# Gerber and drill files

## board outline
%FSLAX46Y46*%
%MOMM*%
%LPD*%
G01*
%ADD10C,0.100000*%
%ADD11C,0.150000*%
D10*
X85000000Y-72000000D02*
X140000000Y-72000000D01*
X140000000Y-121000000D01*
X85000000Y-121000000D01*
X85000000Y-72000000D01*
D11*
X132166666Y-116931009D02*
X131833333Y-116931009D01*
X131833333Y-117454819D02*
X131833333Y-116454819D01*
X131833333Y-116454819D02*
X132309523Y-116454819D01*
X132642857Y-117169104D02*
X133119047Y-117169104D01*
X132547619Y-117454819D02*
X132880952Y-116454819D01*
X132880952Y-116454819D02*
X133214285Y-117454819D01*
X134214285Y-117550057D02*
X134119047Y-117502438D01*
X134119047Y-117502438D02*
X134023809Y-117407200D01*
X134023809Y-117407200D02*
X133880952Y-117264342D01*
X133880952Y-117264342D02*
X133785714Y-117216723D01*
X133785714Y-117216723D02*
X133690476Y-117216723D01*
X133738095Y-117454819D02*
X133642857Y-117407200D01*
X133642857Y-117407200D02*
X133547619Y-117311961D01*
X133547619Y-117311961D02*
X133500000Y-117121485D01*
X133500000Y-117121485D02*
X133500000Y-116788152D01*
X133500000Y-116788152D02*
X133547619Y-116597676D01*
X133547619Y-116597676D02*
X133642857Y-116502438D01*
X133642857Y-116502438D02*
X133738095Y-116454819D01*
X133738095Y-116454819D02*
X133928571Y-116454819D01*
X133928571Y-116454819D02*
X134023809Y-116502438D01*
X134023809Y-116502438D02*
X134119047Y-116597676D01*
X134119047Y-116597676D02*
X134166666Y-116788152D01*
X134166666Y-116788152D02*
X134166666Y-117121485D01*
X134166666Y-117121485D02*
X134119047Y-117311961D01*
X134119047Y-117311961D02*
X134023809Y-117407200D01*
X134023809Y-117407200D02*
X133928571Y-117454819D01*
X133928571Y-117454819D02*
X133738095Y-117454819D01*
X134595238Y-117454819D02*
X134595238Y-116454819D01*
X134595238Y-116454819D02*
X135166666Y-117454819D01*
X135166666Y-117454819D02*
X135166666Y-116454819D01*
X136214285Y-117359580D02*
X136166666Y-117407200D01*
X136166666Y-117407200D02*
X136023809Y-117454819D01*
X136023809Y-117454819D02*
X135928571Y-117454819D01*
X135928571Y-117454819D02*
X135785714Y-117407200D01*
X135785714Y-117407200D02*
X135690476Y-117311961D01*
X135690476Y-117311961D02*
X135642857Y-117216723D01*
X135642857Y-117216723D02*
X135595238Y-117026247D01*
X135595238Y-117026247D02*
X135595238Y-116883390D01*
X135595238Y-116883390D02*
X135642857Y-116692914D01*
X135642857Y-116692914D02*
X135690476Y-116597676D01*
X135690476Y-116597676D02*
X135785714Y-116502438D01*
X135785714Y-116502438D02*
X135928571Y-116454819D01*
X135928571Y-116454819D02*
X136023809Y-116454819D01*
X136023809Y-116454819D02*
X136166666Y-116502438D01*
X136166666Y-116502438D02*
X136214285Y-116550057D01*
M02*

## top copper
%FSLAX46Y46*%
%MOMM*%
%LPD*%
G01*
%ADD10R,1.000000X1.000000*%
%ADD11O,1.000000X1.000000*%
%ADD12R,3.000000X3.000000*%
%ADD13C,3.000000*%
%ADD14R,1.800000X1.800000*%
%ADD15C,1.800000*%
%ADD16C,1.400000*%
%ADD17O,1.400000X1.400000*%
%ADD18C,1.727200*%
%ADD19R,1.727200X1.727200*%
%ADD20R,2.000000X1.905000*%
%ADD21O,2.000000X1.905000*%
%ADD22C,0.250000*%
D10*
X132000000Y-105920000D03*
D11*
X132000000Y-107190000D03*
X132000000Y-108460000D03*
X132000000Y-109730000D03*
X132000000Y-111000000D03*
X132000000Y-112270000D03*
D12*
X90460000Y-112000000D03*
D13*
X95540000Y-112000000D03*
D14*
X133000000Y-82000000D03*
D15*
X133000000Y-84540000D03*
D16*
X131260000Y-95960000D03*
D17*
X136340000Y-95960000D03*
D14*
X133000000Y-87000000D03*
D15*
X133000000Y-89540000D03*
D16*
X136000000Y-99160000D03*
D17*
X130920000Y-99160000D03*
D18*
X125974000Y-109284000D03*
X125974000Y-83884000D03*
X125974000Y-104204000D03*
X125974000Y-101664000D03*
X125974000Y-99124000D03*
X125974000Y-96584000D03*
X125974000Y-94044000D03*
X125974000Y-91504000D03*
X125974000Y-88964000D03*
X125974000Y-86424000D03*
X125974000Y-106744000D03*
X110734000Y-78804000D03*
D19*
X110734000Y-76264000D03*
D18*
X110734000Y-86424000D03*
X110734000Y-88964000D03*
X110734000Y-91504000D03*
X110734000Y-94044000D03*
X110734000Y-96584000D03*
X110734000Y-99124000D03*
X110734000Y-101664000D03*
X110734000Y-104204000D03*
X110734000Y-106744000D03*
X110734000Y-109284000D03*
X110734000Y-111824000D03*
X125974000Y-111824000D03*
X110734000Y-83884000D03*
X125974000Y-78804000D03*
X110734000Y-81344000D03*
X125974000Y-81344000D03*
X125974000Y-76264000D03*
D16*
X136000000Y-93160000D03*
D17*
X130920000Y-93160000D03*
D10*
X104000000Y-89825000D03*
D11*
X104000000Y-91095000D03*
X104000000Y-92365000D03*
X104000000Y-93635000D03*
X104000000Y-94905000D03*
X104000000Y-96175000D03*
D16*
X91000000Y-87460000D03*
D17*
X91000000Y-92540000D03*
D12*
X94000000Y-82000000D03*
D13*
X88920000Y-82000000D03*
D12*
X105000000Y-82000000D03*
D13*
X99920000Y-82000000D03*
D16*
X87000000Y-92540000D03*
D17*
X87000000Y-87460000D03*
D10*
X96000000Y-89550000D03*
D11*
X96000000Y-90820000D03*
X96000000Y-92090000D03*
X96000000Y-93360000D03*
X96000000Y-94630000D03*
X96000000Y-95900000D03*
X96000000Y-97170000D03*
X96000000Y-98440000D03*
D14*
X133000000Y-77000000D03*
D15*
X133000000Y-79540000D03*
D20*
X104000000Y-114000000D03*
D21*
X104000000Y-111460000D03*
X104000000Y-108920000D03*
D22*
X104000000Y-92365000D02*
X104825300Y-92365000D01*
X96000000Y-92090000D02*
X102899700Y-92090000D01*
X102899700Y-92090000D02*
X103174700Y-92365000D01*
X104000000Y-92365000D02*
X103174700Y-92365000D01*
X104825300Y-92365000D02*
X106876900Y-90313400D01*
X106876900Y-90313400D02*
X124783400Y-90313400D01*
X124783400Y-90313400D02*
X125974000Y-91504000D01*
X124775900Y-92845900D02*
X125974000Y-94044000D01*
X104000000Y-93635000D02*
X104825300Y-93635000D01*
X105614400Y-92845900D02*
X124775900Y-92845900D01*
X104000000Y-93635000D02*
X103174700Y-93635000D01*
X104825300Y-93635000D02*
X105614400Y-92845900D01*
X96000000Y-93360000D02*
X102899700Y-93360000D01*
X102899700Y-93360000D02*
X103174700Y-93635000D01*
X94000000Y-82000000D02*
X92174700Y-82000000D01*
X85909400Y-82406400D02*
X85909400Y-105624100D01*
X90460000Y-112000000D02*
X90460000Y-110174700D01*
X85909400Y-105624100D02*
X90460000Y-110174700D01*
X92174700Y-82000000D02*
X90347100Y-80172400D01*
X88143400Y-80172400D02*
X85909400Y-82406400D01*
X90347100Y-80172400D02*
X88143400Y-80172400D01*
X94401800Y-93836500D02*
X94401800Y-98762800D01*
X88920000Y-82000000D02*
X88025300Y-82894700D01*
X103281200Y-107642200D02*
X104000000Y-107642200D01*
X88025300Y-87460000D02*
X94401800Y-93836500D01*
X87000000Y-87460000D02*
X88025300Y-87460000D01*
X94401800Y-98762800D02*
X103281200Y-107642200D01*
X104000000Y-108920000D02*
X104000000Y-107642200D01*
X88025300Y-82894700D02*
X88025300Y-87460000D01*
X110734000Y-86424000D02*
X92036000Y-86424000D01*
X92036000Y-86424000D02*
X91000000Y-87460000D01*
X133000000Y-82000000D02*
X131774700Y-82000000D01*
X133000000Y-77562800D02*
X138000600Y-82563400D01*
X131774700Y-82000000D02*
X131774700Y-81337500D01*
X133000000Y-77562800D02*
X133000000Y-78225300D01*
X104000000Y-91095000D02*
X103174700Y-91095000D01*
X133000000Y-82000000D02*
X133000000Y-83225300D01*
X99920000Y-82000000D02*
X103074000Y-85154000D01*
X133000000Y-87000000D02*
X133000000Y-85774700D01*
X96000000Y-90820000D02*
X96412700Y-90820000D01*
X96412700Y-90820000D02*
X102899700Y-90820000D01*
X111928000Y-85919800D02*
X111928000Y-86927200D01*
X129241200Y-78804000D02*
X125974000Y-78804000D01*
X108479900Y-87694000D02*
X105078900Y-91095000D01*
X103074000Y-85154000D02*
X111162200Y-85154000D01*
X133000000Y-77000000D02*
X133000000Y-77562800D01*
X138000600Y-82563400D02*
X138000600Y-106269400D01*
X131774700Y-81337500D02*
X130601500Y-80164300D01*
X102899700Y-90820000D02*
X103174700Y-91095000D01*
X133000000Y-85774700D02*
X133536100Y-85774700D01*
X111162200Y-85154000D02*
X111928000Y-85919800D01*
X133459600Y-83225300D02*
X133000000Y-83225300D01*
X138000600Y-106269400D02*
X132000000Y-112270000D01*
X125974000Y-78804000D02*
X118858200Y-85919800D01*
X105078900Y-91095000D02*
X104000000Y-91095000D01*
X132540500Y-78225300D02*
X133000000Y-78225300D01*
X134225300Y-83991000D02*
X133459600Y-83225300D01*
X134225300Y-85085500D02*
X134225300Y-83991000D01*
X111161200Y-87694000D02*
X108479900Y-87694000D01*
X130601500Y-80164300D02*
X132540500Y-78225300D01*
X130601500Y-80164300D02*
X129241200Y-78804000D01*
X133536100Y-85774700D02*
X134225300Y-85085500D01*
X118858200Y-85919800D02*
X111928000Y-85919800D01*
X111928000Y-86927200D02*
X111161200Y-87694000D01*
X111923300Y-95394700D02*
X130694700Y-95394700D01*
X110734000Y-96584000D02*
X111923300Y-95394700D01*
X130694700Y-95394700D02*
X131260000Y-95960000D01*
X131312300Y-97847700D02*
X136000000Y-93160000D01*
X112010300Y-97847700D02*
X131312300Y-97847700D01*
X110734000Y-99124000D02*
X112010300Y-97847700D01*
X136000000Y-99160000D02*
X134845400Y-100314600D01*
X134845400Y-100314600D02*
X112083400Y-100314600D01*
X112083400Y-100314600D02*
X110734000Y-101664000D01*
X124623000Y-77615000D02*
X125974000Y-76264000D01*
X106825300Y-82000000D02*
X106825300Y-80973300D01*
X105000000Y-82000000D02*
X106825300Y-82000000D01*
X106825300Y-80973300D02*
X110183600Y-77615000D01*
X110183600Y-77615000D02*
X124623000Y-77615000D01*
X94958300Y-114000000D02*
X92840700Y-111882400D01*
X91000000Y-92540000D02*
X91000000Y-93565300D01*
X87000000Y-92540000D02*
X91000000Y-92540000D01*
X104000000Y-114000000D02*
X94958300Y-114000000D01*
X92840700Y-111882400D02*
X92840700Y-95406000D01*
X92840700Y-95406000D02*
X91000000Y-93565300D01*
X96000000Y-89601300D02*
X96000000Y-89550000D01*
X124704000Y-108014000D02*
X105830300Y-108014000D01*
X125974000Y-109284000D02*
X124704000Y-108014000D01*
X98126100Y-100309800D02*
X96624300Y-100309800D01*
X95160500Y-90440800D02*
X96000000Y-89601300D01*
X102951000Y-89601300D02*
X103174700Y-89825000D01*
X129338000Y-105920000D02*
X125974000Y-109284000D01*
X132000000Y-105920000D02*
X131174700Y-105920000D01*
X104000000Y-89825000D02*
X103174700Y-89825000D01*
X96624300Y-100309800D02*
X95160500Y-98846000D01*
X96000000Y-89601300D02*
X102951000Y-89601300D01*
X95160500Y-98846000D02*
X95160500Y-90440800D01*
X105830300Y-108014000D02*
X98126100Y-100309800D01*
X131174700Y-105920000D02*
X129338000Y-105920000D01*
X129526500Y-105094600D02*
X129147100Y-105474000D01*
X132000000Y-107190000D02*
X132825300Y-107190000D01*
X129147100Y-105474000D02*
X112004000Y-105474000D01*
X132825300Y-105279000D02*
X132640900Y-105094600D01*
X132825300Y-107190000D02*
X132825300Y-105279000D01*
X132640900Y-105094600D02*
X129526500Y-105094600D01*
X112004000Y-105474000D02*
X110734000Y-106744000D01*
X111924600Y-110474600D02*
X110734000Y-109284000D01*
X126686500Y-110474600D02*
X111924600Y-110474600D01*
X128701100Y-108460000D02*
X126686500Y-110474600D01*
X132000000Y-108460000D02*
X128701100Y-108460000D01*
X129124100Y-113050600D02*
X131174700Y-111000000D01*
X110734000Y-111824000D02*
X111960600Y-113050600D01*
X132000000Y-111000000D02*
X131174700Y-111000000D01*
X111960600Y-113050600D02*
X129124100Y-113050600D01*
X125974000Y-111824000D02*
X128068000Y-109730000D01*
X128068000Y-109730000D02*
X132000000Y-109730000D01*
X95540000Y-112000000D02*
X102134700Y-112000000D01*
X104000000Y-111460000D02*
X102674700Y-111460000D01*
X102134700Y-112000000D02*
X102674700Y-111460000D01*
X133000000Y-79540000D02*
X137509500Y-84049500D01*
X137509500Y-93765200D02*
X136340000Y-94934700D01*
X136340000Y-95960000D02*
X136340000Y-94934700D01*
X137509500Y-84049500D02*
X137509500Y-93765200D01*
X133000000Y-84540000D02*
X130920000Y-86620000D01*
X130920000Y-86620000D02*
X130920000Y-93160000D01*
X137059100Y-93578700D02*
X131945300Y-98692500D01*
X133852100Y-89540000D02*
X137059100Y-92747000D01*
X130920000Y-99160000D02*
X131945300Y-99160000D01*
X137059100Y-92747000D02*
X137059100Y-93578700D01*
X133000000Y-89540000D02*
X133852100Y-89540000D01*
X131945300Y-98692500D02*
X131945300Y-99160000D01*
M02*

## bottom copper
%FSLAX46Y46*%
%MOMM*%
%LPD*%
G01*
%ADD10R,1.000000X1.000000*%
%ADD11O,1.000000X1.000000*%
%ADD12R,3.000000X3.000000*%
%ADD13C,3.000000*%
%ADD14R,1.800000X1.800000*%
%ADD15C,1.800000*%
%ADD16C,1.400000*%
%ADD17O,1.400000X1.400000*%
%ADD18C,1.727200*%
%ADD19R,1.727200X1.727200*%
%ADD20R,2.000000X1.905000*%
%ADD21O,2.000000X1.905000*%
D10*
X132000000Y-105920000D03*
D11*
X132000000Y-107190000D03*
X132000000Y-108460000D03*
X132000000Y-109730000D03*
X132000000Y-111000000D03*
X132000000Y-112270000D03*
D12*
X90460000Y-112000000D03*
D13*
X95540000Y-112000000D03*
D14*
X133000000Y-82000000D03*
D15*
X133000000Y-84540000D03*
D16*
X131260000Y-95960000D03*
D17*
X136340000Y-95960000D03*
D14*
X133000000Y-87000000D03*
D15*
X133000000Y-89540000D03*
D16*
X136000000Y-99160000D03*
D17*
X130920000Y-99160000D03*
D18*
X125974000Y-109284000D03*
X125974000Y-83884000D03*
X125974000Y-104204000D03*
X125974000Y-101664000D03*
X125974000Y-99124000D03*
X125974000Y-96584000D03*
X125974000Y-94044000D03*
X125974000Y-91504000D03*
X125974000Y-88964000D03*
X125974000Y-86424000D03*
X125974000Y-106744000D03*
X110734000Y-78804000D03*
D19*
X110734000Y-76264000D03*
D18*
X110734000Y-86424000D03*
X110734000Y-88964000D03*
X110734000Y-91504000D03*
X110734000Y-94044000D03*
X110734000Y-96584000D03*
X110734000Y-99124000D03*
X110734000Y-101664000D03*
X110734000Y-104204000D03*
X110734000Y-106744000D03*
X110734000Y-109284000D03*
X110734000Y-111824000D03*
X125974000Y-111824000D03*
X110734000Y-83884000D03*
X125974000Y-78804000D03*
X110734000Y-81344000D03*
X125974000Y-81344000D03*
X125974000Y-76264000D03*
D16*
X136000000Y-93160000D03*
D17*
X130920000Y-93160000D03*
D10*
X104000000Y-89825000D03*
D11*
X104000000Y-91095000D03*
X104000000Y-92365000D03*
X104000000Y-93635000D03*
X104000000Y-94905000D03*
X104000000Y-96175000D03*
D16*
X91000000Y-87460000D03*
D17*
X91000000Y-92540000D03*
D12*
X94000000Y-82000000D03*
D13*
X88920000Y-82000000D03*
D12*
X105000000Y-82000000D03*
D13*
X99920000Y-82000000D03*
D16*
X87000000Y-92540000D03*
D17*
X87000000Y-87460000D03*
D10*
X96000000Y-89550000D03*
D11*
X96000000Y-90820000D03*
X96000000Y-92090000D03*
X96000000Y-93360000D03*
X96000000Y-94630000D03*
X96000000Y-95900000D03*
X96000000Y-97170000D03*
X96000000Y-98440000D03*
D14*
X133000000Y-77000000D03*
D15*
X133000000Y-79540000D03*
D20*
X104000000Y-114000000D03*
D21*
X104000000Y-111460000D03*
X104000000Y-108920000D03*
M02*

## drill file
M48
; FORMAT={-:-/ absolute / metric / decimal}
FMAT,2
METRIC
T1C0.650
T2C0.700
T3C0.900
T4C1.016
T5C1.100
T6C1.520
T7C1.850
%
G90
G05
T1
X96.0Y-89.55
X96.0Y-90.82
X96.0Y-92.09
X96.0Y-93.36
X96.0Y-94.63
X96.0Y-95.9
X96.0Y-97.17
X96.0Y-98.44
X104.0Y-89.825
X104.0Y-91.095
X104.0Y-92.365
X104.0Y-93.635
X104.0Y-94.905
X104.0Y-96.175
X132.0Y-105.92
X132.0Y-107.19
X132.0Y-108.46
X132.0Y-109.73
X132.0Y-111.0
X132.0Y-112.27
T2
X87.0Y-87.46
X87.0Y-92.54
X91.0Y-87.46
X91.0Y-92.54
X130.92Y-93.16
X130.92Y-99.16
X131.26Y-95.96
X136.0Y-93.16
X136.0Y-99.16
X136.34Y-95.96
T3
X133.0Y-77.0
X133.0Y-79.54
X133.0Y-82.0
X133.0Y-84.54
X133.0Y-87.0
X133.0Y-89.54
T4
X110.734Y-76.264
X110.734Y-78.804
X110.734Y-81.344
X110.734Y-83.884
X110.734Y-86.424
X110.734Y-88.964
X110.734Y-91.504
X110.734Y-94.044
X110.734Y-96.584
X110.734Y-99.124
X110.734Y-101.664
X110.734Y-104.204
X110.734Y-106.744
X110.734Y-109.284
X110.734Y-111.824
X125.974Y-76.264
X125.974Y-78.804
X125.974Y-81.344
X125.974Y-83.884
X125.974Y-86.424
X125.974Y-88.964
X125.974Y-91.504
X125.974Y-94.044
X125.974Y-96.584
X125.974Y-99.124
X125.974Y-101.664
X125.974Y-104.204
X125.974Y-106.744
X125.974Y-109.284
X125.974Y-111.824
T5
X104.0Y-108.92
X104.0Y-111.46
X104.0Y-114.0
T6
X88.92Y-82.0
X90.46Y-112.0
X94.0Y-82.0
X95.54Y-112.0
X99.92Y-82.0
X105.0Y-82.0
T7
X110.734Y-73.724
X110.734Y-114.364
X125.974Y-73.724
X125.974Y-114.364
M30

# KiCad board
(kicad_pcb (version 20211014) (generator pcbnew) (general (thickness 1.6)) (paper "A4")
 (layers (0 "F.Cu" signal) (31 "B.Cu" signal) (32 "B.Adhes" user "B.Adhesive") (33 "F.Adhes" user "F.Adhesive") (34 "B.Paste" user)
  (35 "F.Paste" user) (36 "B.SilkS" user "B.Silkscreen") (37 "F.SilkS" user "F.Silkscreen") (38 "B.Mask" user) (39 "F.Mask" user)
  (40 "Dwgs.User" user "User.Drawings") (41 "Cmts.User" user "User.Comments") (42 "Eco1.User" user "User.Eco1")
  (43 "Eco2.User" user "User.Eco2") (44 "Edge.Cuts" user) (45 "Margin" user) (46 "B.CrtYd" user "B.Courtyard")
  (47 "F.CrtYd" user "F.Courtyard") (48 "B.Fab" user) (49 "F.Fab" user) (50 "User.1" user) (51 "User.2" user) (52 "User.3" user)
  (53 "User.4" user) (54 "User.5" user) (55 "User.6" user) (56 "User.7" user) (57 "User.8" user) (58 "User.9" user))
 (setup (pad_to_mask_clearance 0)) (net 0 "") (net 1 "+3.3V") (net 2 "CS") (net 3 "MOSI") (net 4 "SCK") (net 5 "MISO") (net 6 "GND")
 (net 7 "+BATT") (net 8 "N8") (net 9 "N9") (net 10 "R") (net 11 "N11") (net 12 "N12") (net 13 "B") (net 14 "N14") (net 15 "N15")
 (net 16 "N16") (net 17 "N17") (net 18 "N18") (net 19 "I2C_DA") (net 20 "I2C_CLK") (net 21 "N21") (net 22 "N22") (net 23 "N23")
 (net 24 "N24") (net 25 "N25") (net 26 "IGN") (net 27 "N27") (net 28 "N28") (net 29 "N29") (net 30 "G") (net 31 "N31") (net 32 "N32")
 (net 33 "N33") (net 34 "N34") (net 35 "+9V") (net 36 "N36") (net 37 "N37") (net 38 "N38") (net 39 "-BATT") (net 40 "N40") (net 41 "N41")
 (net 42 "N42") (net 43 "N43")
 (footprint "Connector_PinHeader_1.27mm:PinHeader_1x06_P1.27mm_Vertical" (layer "F.Cu") (at 132 105.92)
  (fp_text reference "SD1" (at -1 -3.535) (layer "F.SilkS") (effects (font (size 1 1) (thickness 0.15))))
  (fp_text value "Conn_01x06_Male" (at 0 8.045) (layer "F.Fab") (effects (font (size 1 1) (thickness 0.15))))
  (pad "1" thru_hole rect (at 0 0) (size 1 1) (drill 0.65) (layers *.Cu *.Mask) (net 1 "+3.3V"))
  (pad "2" thru_hole oval (at 0 1.27) (size 1 1) (drill 0.65) (layers *.Cu *.Mask) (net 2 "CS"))
  (pad "3" thru_hole oval (at 0 2.54) (size 1 1) (drill 0.65) (layers *.Cu *.Mask) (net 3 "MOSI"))
  (pad "4" thru_hole oval (at 0 3.81) (size 1 1) (drill 0.65) (layers *.Cu *.Mask) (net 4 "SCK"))
  (pad "5" thru_hole oval (at 0 5.08) (size 1 1) (drill 0.65) (layers *.Cu *.Mask) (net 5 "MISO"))
  (pad "6" thru_hole oval (at 0 6.35) (size 1 1) (drill 0.65) (layers *.Cu *.Mask) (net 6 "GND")))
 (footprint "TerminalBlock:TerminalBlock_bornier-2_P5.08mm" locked (layer "F.Cu") (at 90.46 112)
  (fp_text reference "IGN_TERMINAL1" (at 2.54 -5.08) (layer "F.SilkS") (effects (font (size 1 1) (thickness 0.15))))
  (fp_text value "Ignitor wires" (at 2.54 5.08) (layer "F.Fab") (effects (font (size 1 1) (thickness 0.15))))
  (pad "1" thru_hole rect locked (at 0 0) (size 3 3) (drill 1.52) (layers *.Cu *.Mask) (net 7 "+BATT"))
  (pad "2" thru_hole circle locked (at 5.08 0) (size 3 3) (drill 1.52) (layers *.Cu *.Mask) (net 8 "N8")))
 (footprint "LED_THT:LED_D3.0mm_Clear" (layer "F.Cu") (at 133 82 -90)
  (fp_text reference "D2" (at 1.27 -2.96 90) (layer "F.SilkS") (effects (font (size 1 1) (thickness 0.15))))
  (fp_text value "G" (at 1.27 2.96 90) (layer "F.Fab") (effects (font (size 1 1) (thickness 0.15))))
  (pad "1" thru_hole rect (at 0 0 270) (size 1.8 1.8) (drill 0.9) (layers *.Cu *.Mask) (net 6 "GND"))
  (pad "2" thru_hole circle (at 2.54 0 270) (size 1.8 1.8) (drill 0.9) (layers *.Cu *.Mask) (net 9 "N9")))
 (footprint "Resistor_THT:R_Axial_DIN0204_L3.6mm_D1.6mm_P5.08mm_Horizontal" (layer "F.Cu") (at 131.26 95.96)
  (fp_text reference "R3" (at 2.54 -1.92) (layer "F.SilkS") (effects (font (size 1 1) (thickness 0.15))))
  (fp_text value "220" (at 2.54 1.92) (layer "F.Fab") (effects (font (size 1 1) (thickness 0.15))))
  (pad "1" thru_hole circle (at 0 0) (size 1.4 1.4) (drill 0.7) (layers *.Cu *.Mask) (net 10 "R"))
  (pad "2" thru_hole oval (at 5.08 0) (size 1.4 1.4) (drill 0.7) (layers *.Cu *.Mask) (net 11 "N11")))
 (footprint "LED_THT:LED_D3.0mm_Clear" (layer "F.Cu") (at 133 87 -90)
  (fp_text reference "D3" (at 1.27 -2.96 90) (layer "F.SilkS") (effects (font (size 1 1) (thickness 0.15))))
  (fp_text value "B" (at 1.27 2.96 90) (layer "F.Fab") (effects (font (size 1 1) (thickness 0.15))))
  (pad "1" thru_hole rect (at 0 0 270) (size 1.8 1.8) (drill 0.9) (layers *.Cu *.Mask) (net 6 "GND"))
  (pad "2" thru_hole circle (at 2.54 0 270) (size 1.8 1.8) (drill 0.9) (layers *.Cu *.Mask) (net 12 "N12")))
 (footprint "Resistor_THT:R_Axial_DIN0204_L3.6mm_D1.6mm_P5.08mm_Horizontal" (layer "F.Cu") (at 136 99.16 180)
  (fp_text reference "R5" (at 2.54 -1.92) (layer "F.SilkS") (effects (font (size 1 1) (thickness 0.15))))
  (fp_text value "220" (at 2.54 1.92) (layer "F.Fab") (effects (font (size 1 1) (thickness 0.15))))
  (pad "1" thru_hole circle (at 0 0 180) (size 1.4 1.4) (drill 0.7) (layers *.Cu *.Mask) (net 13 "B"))
  (pad "2" thru_hole oval (at 5.08 0 180) (size 1.4 1.4) (drill 0.7) (layers *.Cu *.Mask) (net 12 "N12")))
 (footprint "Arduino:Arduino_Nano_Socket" (layer "F.Cu") (at 118.354 115.634)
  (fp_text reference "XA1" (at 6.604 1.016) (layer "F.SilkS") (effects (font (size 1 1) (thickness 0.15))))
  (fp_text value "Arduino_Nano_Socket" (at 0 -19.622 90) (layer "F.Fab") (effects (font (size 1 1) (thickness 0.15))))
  (pad "" np_thru_hole circle locked (at 7.62 -41.91) (size 1.85 1.85) (drill 1.85) (layers *.Cu *.Mask))
  (pad "" np_thru_hole circle locked (at 7.62 -1.27) (size 1.85 1.85) (drill 1.85) (layers *.Cu *.Mask))
  (pad "" np_thru_hole circle locked (at -7.62 -41.91) (size 1.85 1.85) (drill 1.85) (layers *.Cu *.Mask))
  (pad "" np_thru_hole circle locked (at -7.62 -1.27) (size 1.85 1.85) (drill 1.85) (layers *.Cu *.Mask))
  (pad "3V3" thru_hole circle locked (at 7.62 -6.35) (size 1.7272 1.7272) (drill 1.016) (layers *.Cu *.Mask) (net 1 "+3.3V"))
  (pad "5V" thru_hole circle locked (at 7.62 -31.75) (size 1.7272 1.7272) (drill 1.016) (layers *.Cu *.Mask) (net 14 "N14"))
  (pad "A0" thru_hole circle locked (at 7.62 -11.43) (size 1.7272 1.7272) (drill 1.016) (layers *.Cu *.Mask) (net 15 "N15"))
  (pad "A1" thru_hole circle locked (at 7.62 -13.97) (size 1.7272 1.7272) (drill 1.016) (layers *.Cu *.Mask) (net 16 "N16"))
  (pad "A2" thru_hole circle locked (at 7.62 -16.51) (size 1.7272 1.7272) (drill 1.016) (layers *.Cu *.Mask) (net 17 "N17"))
  (pad "A3" thru_hole circle locked (at 7.62 -19.05) (size 1.7272 1.7272) (drill 1.016) (layers *.Cu *.Mask) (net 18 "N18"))
  (pad "A4" thru_hole circle locked (at 7.62 -21.59) (size 1.7272 1.7272) (drill 1.016) (layers *.Cu *.Mask) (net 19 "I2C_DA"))
  (pad "A5" thru_hole circle locked (at 7.62 -24.13) (size 1.7272 1.7272) (drill 1.016) (layers *.Cu *.Mask) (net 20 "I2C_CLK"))
  (pad "A6" thru_hole circle locked (at 7.62 -26.67) (size 1.7272 1.7272) (drill 1.016) (layers *.Cu *.Mask) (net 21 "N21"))
  (pad "A7" thru_hole circle locked (at 7.62 -29.21) (size 1.7272 1.7272) (drill 1.016) (layers *.Cu *.Mask) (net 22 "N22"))
  (pad "AREF" thru_hole circle locked (at 7.62 -8.89) (size 1.7272 1.7272) (drill 1.016) (layers *.Cu *.Mask) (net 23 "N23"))
  (pad "D0" thru_hole circle locked (at -7.62 -36.83) (size 1.7272 1.7272) (drill 1.016) (layers *.Cu *.Mask) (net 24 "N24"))
  (pad "D1" thru_hole rect locked (at -7.62 -39.37) (size 1.7272 1.7272) (drill 1.016) (layers *.Cu *.Mask) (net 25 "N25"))
  (pad "D2" thru_hole circle locked (at -7.62 -29.21) (size 1.7272 1.7272) (drill 1.016) (layers *.Cu *.Mask) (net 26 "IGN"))
  (pad "D3" thru_hole circle locked (at -7.62 -26.67) (size 1.7272 1.7272) (drill 1.016) (layers *.Cu *.Mask) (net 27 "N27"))
  (pad "D4" thru_hole circle locked (at -7.62 -24.13) (size 1.7272 1.7272) (drill 1.016) (layers *.Cu *.Mask) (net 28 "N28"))
  (pad "D5" thru_hole circle locked (at -7.62 -21.59) (size 1.7272 1.7272) (drill 1.016) (layers *.Cu *.Mask) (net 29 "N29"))
  (pad "D6" thru_hole circle locked (at -7.62 -19.05) (size 1.7272 1.7272) (drill 1.016) (layers *.Cu *.Mask) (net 10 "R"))
  (pad "D7" thru_hole circle locked (at -7.62 -16.51) (size 1.7272 1.7272) (drill 1.016) (layers *.Cu *.Mask) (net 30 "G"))
  (pad "D8" thru_hole circle locked (at -7.62 -13.97) (size 1.7272 1.7272) (drill 1.016) (layers *.Cu *.Mask) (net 13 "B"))
  (pad "D9" thru_hole circle locked (at -7.62 -11.43) (size 1.7272 1.7272) (drill 1.016) (layers *.Cu *.Mask) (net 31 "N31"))
  (pad "D10" thru_hole circle locked (at -7.62 -8.89) (size 1.7272 1.7272) (drill 1.016) (layers *.Cu *.Mask) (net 2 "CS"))
  (pad "D11" thru_hole circle locked (at -7.62 -6.35) (size 1.7272 1.7272) (drill 1.016) (layers *.Cu *.Mask) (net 3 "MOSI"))
  (pad "D12" thru_hole circle locked (at -7.62 -3.81) (size 1.7272 1.7272) (drill 1.016) (layers *.Cu *.Mask) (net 5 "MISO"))
  (pad "D13" thru_hole circle locked (at 7.62 -3.81) (size 1.7272 1.7272) (drill 1.016) (layers *.Cu *.Mask) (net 4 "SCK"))
  (pad "GND1" thru_hole circle locked (at -7.62 -31.75) (size 1.7272 1.7272) (drill 1.016) (layers *.Cu *.Mask) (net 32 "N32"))
  (pad "GND2" thru_hole circle locked (at 7.62 -36.83) (size 1.7272 1.7272) (drill 1.016) (layers *.Cu *.Mask) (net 6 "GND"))
  (pad "RST1" thru_hole circle locked (at -7.62 -34.29) (size 1.7272 1.7272) (drill 1.016) (layers *.Cu *.Mask) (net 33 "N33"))
  (pad "RST2" thru_hole circle locked (at 7.62 -34.29) (size 1.7272 1.7272) (drill 1.016) (layers *.Cu *.Mask) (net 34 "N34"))
  (pad "VIN" thru_hole circle locked (at 7.62 -39.37) (size 1.7272 1.7272) (drill 1.016) (layers *.Cu *.Mask) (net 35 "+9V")))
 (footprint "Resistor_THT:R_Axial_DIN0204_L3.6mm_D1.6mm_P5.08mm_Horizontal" (layer "F.Cu") (at 136 93.16 180)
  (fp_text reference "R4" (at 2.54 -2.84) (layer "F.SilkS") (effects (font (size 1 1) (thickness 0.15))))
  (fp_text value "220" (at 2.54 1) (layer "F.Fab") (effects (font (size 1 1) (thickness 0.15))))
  (pad "1" thru_hole circle (at 0 0 180) (size 1.4 1.4) (drill 0.7) (layers *.Cu *.Mask) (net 30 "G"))
  (pad "2" thru_hole oval (at 5.08 0 180) (size 1.4 1.4) (drill 0.7) (layers *.Cu *.Mask) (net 9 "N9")))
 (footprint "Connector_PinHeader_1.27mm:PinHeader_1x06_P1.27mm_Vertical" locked (layer "F.Cu") (at 104 89.825)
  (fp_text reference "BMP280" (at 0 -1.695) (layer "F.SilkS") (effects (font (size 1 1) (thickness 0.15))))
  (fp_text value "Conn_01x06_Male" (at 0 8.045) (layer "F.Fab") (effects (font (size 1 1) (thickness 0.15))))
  (pad "1" thru_hole rect locked (at 0 0) (size 1 1) (drill 0.65) (layers *.Cu *.Mask) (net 1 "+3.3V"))
  (pad "2" thru_hole oval locked (at 0 1.27) (size 1 1) (drill 0.65) (layers *.Cu *.Mask) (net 6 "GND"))
  (pad "3" thru_hole oval locked (at 0 2.54) (size 1 1) (drill 0.65) (layers *.Cu *.Mask) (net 20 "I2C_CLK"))
  (pad "4" thru_hole oval locked (at 0 3.81) (size 1 1) (drill 0.65) (layers *.Cu *.Mask) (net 19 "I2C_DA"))
  (pad "5" thru_hole oval locked (at 0 5.08) (size 1 1) (drill 0.65) (layers *.Cu *.Mask) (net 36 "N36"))
  (pad "6" thru_hole oval locked (at 0 6.35) (size 1 1) (drill 0.65) (layers *.Cu *.Mask) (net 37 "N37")))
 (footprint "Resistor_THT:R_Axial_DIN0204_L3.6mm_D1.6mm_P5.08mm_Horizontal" (layer "F.Cu") (at 91 87.46 -90)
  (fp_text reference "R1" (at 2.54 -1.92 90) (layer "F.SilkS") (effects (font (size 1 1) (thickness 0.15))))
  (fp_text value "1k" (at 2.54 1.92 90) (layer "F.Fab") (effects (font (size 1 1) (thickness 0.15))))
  (pad "1" thru_hole circle (at 0 0 270) (size 1.4 1.4) (drill 0.7) (layers *.Cu *.Mask) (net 26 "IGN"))
  (pad "2" thru_hole oval (at 5.08 0 270) (size 1.4 1.4) (drill 0.7) (layers *.Cu *.Mask) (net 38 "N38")))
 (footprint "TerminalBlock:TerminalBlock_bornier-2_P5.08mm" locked (layer "F.Cu") (at 94 82 180)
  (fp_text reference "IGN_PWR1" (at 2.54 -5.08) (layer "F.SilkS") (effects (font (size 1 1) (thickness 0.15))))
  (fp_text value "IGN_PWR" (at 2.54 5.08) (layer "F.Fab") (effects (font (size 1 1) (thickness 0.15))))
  (pad "1" thru_hole rect locked (at 0 0 180) (size 3 3) (drill 1.52) (layers *.Cu *.Mask) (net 7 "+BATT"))
  (pad "2" thru_hole circle locked (at 5.08 0 180) (size 3 3) (drill 1.52) (layers *.Cu *.Mask) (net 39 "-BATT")))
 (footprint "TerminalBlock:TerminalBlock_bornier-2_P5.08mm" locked (layer "F.Cu") (at 105 82 180)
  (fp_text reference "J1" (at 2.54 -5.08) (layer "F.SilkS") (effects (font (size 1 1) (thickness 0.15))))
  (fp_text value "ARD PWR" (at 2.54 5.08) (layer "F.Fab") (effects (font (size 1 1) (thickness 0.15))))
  (pad "1" thru_hole rect locked (at 0 0 180) (size 3 3) (drill 1.52) (layers *.Cu *.Mask) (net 35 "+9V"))
  (pad "2" thru_hole circle locked (at 5.08 0 180) (size 3 3) (drill 1.52) (layers *.Cu *.Mask) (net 6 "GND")))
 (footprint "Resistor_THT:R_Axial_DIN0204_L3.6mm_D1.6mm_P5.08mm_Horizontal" (layer "F.Cu") (at 87 92.54 90)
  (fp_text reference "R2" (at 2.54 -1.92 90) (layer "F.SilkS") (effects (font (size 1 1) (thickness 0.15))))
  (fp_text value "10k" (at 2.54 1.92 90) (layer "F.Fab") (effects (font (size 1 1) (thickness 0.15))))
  (pad "1" thru_hole circle (at 0 0 90) (size 1.4 1.4) (drill 0.7) (layers *.Cu *.Mask) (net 38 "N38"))
  (pad "2" thru_hole oval (at 5.08 0 90) (size 1.4 1.4) (drill 0.7) (layers *.Cu *.Mask) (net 39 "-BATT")))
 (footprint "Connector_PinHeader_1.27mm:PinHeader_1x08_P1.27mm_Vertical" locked (layer "F.Cu") (at 96 89.55)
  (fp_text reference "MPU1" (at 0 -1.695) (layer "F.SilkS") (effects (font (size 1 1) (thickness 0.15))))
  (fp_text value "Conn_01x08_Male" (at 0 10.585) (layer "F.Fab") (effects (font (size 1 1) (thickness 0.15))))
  (pad "1" thru_hole rect locked (at 0 0) (size 1 1) (drill 0.65) (layers *.Cu *.Mask) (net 1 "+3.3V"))
  (pad "2" thru_hole oval locked (at 0 1.27) (size 1 1) (drill 0.65) (layers *.Cu *.Mask) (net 6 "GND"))
  (pad "3" thru_hole oval locked (at 0 2.54) (size 1 1) (drill 0.65) (layers *.Cu *.Mask) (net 20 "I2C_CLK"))
  (pad "4" thru_hole oval locked (at 0 3.81) (size 1 1) (drill 0.65) (layers *.Cu *.Mask) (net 19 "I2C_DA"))
  (pad "5" thru_hole oval locked (at 0 5.08) (size 1 1) (drill 0.65) (layers *.Cu *.Mask) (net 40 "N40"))
  (pad "6" thru_hole oval locked (at 0 6.35) (size 1 1) (drill 0.65) (layers *.Cu *.Mask) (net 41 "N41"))
  (pad "7" thru_hole oval locked (at 0 7.62) (size 1 1) (drill 0.65) (layers *.Cu *.Mask) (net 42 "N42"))
  (pad "8" thru_hole oval locked (at 0 8.89) (size 1 1) (drill 0.65) (layers *.Cu *.Mask) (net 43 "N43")))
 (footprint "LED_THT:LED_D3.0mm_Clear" (layer "F.Cu") (at 133 77 -90)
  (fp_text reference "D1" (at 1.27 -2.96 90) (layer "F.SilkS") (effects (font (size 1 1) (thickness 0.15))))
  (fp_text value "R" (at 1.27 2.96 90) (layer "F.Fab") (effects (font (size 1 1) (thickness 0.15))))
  (pad "1" thru_hole rect (at 0 0 270) (size 1.8 1.8) (drill 0.9) (layers *.Cu *.Mask) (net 6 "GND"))
  (pad "2" thru_hole circle (at 2.54 0 270) (size 1.8 1.8) (drill 0.9) (layers *.Cu *.Mask) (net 11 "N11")))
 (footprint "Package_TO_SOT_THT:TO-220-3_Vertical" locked (layer "F.Cu") (at 104 114 90)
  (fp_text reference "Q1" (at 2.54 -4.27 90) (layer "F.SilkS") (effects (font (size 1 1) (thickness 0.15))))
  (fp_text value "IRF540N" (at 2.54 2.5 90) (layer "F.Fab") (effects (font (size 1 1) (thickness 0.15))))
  (pad "1" thru_hole rect locked (at 0 0 90) (size 1.905 2) (drill 1.1) (layers *.Cu *.Mask) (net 38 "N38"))
  (pad "2" thru_hole oval locked (at 2.54 0 90) (size 1.905 2) (drill 1.1) (layers *.Cu *.Mask) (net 8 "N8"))
  (pad "3" thru_hole oval locked (at 5.08 0 90) (size 1.905 2) (drill 1.1) (layers *.Cu *.Mask) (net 39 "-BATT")))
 (gr_rect (start 85 72) (end 140 121) (layer "Edge.Cuts") (width 0.1) (fill none))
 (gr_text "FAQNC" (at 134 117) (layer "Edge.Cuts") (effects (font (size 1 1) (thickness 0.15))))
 (segment (start 104 92.365) (end 104.8253 92.365) (width 0.25) (layer "F.Cu") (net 20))
 (segment (start 96 92.09) (end 102.8997 92.09) (width 0.25) (layer "F.Cu") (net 20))
 (segment (start 102.8997 92.09) (end 103.1747 92.365) (width 0.25) (layer "F.Cu") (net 20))
 (segment (start 104 92.365) (end 103.1747 92.365) (width 0.25) (layer "F.Cu") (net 20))
 (segment (start 104.8253 92.365) (end 106.8769 90.3134) (width 0.25) (layer "F.Cu") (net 20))
 (segment (start 106.8769 90.3134) (end 124.7834 90.3134) (width 0.25) (layer "F.Cu") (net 20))
 (segment (start 124.7834 90.3134) (end 125.974 91.504) (width 0.25) (layer "F.Cu") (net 20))
 (segment (start 124.7759 92.8459) (end 125.974 94.044) (width 0.25) (layer "F.Cu") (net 19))
 (segment (start 104 93.635) (end 104.8253 93.635) (width 0.25) (layer "F.Cu") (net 19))
 (segment (start 105.6144 92.8459) (end 124.7759 92.8459) (width 0.25) (layer "F.Cu") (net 19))
 (segment (start 104 93.635) (end 103.1747 93.635) (width 0.25) (layer "F.Cu") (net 19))
 (segment (start 104.8253 93.635) (end 105.6144 92.8459) (width 0.25) (layer "F.Cu") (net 19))
 (segment (start 96 93.36) (end 102.8997 93.36) (width 0.25) (layer "F.Cu") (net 19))
 (segment (start 102.8997 93.36) (end 103.1747 93.635) (width 0.25) (layer "F.Cu") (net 19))
 (segment (start 94 82) (end 92.1747 82) (width 0.25) (layer "F.Cu") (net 7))
 (segment (start 85.9094 82.4064) (end 85.9094 105.6241) (width 0.25) (layer "F.Cu") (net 7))
 (segment (start 90.46 112) (end 90.46 110.1747) (width 0.25) (layer "F.Cu") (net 7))
 (segment (start 85.9094 105.6241) (end 90.46 110.1747) (width 0.25) (layer "F.Cu") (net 7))
 (segment (start 92.1747 82) (end 90.3471 80.1724) (width 0.25) (layer "F.Cu") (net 7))
 (segment (start 88.1434 80.1724) (end 85.9094 82.4064) (width 0.25) (layer "F.Cu") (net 7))
 (segment (start 90.3471 80.1724) (end 88.1434 80.1724) (width 0.25) (layer "F.Cu") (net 7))
 (segment (start 94.4018 93.8365) (end 94.4018 98.7628) (width 0.25) (layer "F.Cu") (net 39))
 (segment (start 88.92 82) (end 88.0253 82.8947) (width 0.25) (layer "F.Cu") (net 39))
 (segment (start 103.2812 107.6422) (end 104 107.6422) (width 0.25) (layer "F.Cu") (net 39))
 (segment (start 88.0253 87.46) (end 94.4018 93.8365) (width 0.25) (layer "F.Cu") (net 39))
 (segment (start 87 87.46) (end 88.0253 87.46) (width 0.25) (layer "F.Cu") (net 39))
 (segment (start 94.4018 98.7628) (end 103.2812 107.6422) (width 0.25) (layer "F.Cu") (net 39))
 (segment (start 104 108.92) (end 104 107.6422) (width 0.25) (layer "F.Cu") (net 39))
 (segment (start 88.0253 82.8947) (end 88.0253 87.46) (width 0.25) (layer "F.Cu") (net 39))
 (segment (start 110.734 86.424) (end 92.036 86.424) (width 0.25) (layer "F.Cu") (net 26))
 (segment (start 92.036 86.424) (end 91 87.46) (width 0.25) (layer "F.Cu") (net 26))
 (segment (start 133 82) (end 131.7747 82) (width 0.25) (layer "F.Cu") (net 6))
 (segment (start 133 77.5628) (end 138.0006 82.5634) (width 0.25) (layer "F.Cu") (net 6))
 (segment (start 131.7747 82) (end 131.7747 81.3375) (width 0.25) (layer "F.Cu") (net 6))
 (segment (start 133 77.5628) (end 133 78.2253) (width 0.25) (layer "F.Cu") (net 6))
 (segment (start 104 91.095) (end 103.1747 91.095) (width 0.25) (layer "F.Cu") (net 6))
 (segment (start 133 82) (end 133 83.2253) (width 0.25) (layer "F.Cu") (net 6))
 (segment (start 99.92 82) (end 103.074 85.154) (width 0.25) (layer "F.Cu") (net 6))
 (segment (start 133 87) (end 133 85.7747) (width 0.25) (layer "F.Cu") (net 6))
 (segment (start 96 90.82) (end 96.4127 90.82) (width 0.25) (layer "F.Cu") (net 6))
 (segment (start 96.4127 90.82) (end 102.8997 90.82) (width 0.25) (layer "F.Cu") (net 6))
 (segment (start 111.928 85.9198) (end 111.928 86.9272) (width 0.25) (layer "F.Cu") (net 6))
 (segment (start 129.2412 78.804) (end 125.974 78.804) (width 0.25) (layer "F.Cu") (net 6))
 (segment (start 108.4799 87.694) (end 105.0789 91.095) (width 0.25) (layer "F.Cu") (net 6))
 (segment (start 103.074 85.154) (end 111.1622 85.154) (width 0.25) (layer "F.Cu") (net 6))
 (segment (start 133 77) (end 133 77.5628) (width 0.25) (layer "F.Cu") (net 6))
 (segment (start 138.0006 82.5634) (end 138.0006 106.2694) (width 0.25) (layer "F.Cu") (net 6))
 (segment (start 131.7747 81.3375) (end 130.6015 80.1643) (width 0.25) (layer "F.Cu") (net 6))
 (segment (start 102.8997 90.82) (end 103.1747 91.095) (width 0.25) (layer "F.Cu") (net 6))
 (segment (start 133 85.7747) (end 133.5361 85.7747) (width 0.25) (layer "F.Cu") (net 6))
 (segment (start 111.1622 85.154) (end 111.928 85.9198) (width 0.25) (layer "F.Cu") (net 6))
 (segment (start 133.4596 83.2253) (end 133 83.2253) (width 0.25) (layer "F.Cu") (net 6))
 (segment (start 138.0006 106.2694) (end 132 112.27) (width 0.25) (layer "F.Cu") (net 6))
 (segment (start 125.974 78.804) (end 118.8582 85.9198) (width 0.25) (layer "F.Cu") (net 6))
 (segment (start 105.0789 91.095) (end 104 91.095) (width 0.25) (layer "F.Cu") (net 6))
 (segment (start 132.5405 78.2253) (end 133 78.2253) (width 0.25) (layer "F.Cu") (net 6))
 (segment (start 134.2253 83.991) (end 133.4596 83.2253) (width 0.25) (layer "F.Cu") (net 6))
 (segment (start 134.2253 85.0855) (end 134.2253 83.991) (width 0.25) (layer "F.Cu") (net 6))
 (segment (start 111.1612 87.694) (end 108.4799 87.694) (width 0.25) (layer "F.Cu") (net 6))
 (segment (start 130.6015 80.1643) (end 132.5405 78.2253) (width 0.25) (layer "F.Cu") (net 6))
 (segment (start 130.6015 80.1643) (end 129.2412 78.804) (width 0.25) (layer "F.Cu") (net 6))
 (segment (start 133.5361 85.7747) (end 134.2253 85.0855) (width 0.25) (layer "F.Cu") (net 6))
 (segment (start 118.8582 85.9198) (end 111.928 85.9198) (width 0.25) (layer "F.Cu") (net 6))
 (segment (start 111.928 86.9272) (end 111.1612 87.694) (width 0.25) (layer "F.Cu") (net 6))
 (segment (start 111.9233 95.3947) (end 130.6947 95.3947) (width 0.25) (layer "F.Cu") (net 10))
 (segment (start 110.734 96.584) (end 111.9233 95.3947) (width 0.25) (layer "F.Cu") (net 10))
 (segment (start 130.6947 95.3947) (end 131.26 95.96) (width 0.25) (layer "F.Cu") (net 10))
 (segment (start 131.3123 97.8477) (end 136 93.16) (width 0.25) (layer "F.Cu") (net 30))
 (segment (start 112.0103 97.8477) (end 131.3123 97.8477) (width 0.25) (layer "F.Cu") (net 30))
 (segment (start 110.734 99.124) (end 112.0103 97.8477) (width 0.25) (layer "F.Cu") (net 30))
 (segment (start 136 99.16) (end 134.8454 100.3146) (width 0.25) (layer "F.Cu") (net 13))
 (segment (start 134.8454 100.3146) (end 112.0834 100.3146) (width 0.25) (layer "F.Cu") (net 13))
 (segment (start 112.0834 100.3146) (end 110.734 101.664) (width 0.25) (layer "F.Cu") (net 13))
 (segment (start 124.623 77.615) (end 125.974 76.264) (width 0.25) (layer "F.Cu") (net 35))
 (segment (start 106.8253 82) (end 106.8253 80.9733) (width 0.25) (layer "F.Cu") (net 35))
 (segment (start 105 82) (end 106.8253 82) (width 0.25) (layer "F.Cu") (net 35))
 (segment (start 106.8253 80.9733) (end 110.1836 77.615) (width 0.25) (layer "F.Cu") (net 35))
 (segment (start 110.1836 77.615) (end 124.623 77.615) (width 0.25) (layer "F.Cu") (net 35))
 (segment (start 94.9583 114) (end 92.8407 111.8824) (width 0.25) (layer "F.Cu") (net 38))
 (segment (start 91 92.54) (end 91 93.5653) (width 0.25) (layer "F.Cu") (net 38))
 (segment (start 87 92.54) (end 91 92.54) (width 0.25) (layer "F.Cu") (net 38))
 (segment (start 104 114) (end 94.9583 114) (width 0.25) (layer "F.Cu") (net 38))
 (segment (start 92.8407 111.8824) (end 92.8407 95.406) (width 0.25) (layer "F.Cu") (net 38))
 (segment (start 92.8407 95.406) (end 91 93.5653) (width 0.25) (layer "F.Cu") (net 38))
 (segment (start 96 89.6013) (end 96 89.55) (width 0.25) (layer "F.Cu") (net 1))
 (segment (start 124.704 108.014) (end 105.8303 108.014) (width 0.25) (layer "F.Cu") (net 1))
 (segment (start 125.974 109.284) (end 124.704 108.014) (width 0.25) (layer "F.Cu") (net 1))
 (segment (start 98.1261 100.3098) (end 96.6243 100.3098) (width 0.25) (layer "F.Cu") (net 1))
 (segment (start 95.1605 90.4408) (end 96 89.6013) (width 0.25) (layer "F.Cu") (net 1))
 (segment (start 102.951 89.6013) (end 103.1747 89.825) (width 0.25) (layer "F.Cu") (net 1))
 (segment (start 129.338 105.92) (end 125.974 109.284) (width 0.25) (layer "F.Cu") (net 1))
 (segment (start 132 105.92) (end 131.1747 105.92) (width 0.25) (layer "F.Cu") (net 1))
 (segment (start 104 89.825) (end 103.1747 89.825) (width 0.25) (layer "F.Cu") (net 1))
 (segment (start 96.6243 100.3098) (end 95.1605 98.846) (width 0.25) (layer "F.Cu") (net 1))
 (segment (start 96 89.6013) (end 102.951 89.6013) (width 0.25) (layer "F.Cu") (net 1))
 (segment (start 95.1605 98.846) (end 95.1605 90.4408) (width 0.25) (layer "F.Cu") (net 1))
 (segment (start 105.8303 108.014) (end 98.1261 100.3098) (width 0.25) (layer "F.Cu") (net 1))
 (segment (start 131.1747 105.92) (end 129.338 105.92) (width 0.25) (layer "F.Cu") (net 1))
 (segment (start 129.5265 105.0946) (end 129.1471 105.474) (width 0.25) (layer "F.Cu") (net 2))
 (segment (start 132 107.19) (end 132.8253 107.19) (width 0.25) (layer "F.Cu") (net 2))
 (segment (start 129.1471 105.474) (end 112.004 105.474) (width 0.25) (layer "F.Cu") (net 2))
 (segment (start 132.8253 105.279) (end 132.6409 105.0946) (width 0.25) (layer "F.Cu") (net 2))
 (segment (start 132.8253 107.19) (end 132.8253 105.279) (width 0.25) (layer "F.Cu") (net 2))
 (segment (start 132.6409 105.0946) (end 129.5265 105.0946) (width 0.25) (layer "F.Cu") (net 2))
 (segment (start 112.004 105.474) (end 110.734 106.744) (width 0.25) (layer "F.Cu") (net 2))
 (segment (start 111.9246 110.4746) (end 110.734 109.284) (width 0.25) (layer "F.Cu") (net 3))
 (segment (start 126.6865 110.4746) (end 111.9246 110.4746) (width 0.25) (layer "F.Cu") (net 3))
 (segment (start 128.7011 108.46) (end 126.6865 110.4746) (width 0.25) (layer "F.Cu") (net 3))
 (segment (start 132 108.46) (end 128.7011 108.46) (width 0.25) (layer "F.Cu") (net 3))
 (segment (start 129.1241 113.0506) (end 131.1747 111) (width 0.25) (layer "F.Cu") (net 5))
 (segment (start 110.734 111.824) (end 111.9606 113.0506) (width 0.25) (layer "F.Cu") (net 5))
 (segment (start 132 111) (end 131.1747 111) (width 0.25) (layer "F.Cu") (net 5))
 (segment (start 111.9606 113.0506) (end 129.1241 113.0506) (width 0.25) (layer "F.Cu") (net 5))
 (segment (start 125.974 111.824) (end 128.068 109.73) (width 0.25) (layer "F.Cu") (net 4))
 (segment (start 128.068 109.73) (end 132 109.73) (width 0.25) (layer "F.Cu") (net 4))
 (segment (start 95.54 112) (end 102.1347 112) (width 0.25) (layer "F.Cu") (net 8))
 (segment (start 104 111.46) (end 102.6747 111.46) (width 0.25) (layer "F.Cu") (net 8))
 (segment (start 102.1347 112) (end 102.6747 111.46) (width 0.25) (layer "F.Cu") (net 8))
 (segment (start 133 79.54) (end 137.5095 84.0495) (width 0.25) (layer "F.Cu") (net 11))
 (segment (start 137.5095 93.7652) (end 136.34 94.9347) (width 0.25) (layer "F.Cu") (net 11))
 (segment (start 136.34 95.96) (end 136.34 94.9347) (width 0.25) (layer "F.Cu") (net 11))
 (segment (start 137.5095 84.0495) (end 137.5095 93.7652) (width 0.25) (layer "F.Cu") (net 11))
 (segment (start 133 84.54) (end 130.92 86.62) (width 0.25) (layer "F.Cu") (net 9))
 (segment (start 130.92 86.62) (end 130.92 93.16) (width 0.25) (layer "F.Cu") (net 9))
 (segment (start 137.0591 93.5787) (end 131.9453 98.6925) (width 0.25) (layer "F.Cu") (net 12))
 (segment (start 133.8521 89.54) (end 137.0591 92.747) (width 0.25) (layer "F.Cu") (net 12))
 (segment (start 130.92 99.16) (end 131.9453 99.16) (width 0.25) (layer "F.Cu") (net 12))
 (segment (start 137.0591 92.747) (end 137.0591 93.5787) (width 0.25) (layer "F.Cu") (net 12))
 (segment (start 133 89.54) (end 133.8521 89.54) (width 0.25) (layer "F.Cu") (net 12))
 (segment (start 131.9453 98.6925) (end 131.9453 99.16) (width 0.25) (layer "F.Cu") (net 12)))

